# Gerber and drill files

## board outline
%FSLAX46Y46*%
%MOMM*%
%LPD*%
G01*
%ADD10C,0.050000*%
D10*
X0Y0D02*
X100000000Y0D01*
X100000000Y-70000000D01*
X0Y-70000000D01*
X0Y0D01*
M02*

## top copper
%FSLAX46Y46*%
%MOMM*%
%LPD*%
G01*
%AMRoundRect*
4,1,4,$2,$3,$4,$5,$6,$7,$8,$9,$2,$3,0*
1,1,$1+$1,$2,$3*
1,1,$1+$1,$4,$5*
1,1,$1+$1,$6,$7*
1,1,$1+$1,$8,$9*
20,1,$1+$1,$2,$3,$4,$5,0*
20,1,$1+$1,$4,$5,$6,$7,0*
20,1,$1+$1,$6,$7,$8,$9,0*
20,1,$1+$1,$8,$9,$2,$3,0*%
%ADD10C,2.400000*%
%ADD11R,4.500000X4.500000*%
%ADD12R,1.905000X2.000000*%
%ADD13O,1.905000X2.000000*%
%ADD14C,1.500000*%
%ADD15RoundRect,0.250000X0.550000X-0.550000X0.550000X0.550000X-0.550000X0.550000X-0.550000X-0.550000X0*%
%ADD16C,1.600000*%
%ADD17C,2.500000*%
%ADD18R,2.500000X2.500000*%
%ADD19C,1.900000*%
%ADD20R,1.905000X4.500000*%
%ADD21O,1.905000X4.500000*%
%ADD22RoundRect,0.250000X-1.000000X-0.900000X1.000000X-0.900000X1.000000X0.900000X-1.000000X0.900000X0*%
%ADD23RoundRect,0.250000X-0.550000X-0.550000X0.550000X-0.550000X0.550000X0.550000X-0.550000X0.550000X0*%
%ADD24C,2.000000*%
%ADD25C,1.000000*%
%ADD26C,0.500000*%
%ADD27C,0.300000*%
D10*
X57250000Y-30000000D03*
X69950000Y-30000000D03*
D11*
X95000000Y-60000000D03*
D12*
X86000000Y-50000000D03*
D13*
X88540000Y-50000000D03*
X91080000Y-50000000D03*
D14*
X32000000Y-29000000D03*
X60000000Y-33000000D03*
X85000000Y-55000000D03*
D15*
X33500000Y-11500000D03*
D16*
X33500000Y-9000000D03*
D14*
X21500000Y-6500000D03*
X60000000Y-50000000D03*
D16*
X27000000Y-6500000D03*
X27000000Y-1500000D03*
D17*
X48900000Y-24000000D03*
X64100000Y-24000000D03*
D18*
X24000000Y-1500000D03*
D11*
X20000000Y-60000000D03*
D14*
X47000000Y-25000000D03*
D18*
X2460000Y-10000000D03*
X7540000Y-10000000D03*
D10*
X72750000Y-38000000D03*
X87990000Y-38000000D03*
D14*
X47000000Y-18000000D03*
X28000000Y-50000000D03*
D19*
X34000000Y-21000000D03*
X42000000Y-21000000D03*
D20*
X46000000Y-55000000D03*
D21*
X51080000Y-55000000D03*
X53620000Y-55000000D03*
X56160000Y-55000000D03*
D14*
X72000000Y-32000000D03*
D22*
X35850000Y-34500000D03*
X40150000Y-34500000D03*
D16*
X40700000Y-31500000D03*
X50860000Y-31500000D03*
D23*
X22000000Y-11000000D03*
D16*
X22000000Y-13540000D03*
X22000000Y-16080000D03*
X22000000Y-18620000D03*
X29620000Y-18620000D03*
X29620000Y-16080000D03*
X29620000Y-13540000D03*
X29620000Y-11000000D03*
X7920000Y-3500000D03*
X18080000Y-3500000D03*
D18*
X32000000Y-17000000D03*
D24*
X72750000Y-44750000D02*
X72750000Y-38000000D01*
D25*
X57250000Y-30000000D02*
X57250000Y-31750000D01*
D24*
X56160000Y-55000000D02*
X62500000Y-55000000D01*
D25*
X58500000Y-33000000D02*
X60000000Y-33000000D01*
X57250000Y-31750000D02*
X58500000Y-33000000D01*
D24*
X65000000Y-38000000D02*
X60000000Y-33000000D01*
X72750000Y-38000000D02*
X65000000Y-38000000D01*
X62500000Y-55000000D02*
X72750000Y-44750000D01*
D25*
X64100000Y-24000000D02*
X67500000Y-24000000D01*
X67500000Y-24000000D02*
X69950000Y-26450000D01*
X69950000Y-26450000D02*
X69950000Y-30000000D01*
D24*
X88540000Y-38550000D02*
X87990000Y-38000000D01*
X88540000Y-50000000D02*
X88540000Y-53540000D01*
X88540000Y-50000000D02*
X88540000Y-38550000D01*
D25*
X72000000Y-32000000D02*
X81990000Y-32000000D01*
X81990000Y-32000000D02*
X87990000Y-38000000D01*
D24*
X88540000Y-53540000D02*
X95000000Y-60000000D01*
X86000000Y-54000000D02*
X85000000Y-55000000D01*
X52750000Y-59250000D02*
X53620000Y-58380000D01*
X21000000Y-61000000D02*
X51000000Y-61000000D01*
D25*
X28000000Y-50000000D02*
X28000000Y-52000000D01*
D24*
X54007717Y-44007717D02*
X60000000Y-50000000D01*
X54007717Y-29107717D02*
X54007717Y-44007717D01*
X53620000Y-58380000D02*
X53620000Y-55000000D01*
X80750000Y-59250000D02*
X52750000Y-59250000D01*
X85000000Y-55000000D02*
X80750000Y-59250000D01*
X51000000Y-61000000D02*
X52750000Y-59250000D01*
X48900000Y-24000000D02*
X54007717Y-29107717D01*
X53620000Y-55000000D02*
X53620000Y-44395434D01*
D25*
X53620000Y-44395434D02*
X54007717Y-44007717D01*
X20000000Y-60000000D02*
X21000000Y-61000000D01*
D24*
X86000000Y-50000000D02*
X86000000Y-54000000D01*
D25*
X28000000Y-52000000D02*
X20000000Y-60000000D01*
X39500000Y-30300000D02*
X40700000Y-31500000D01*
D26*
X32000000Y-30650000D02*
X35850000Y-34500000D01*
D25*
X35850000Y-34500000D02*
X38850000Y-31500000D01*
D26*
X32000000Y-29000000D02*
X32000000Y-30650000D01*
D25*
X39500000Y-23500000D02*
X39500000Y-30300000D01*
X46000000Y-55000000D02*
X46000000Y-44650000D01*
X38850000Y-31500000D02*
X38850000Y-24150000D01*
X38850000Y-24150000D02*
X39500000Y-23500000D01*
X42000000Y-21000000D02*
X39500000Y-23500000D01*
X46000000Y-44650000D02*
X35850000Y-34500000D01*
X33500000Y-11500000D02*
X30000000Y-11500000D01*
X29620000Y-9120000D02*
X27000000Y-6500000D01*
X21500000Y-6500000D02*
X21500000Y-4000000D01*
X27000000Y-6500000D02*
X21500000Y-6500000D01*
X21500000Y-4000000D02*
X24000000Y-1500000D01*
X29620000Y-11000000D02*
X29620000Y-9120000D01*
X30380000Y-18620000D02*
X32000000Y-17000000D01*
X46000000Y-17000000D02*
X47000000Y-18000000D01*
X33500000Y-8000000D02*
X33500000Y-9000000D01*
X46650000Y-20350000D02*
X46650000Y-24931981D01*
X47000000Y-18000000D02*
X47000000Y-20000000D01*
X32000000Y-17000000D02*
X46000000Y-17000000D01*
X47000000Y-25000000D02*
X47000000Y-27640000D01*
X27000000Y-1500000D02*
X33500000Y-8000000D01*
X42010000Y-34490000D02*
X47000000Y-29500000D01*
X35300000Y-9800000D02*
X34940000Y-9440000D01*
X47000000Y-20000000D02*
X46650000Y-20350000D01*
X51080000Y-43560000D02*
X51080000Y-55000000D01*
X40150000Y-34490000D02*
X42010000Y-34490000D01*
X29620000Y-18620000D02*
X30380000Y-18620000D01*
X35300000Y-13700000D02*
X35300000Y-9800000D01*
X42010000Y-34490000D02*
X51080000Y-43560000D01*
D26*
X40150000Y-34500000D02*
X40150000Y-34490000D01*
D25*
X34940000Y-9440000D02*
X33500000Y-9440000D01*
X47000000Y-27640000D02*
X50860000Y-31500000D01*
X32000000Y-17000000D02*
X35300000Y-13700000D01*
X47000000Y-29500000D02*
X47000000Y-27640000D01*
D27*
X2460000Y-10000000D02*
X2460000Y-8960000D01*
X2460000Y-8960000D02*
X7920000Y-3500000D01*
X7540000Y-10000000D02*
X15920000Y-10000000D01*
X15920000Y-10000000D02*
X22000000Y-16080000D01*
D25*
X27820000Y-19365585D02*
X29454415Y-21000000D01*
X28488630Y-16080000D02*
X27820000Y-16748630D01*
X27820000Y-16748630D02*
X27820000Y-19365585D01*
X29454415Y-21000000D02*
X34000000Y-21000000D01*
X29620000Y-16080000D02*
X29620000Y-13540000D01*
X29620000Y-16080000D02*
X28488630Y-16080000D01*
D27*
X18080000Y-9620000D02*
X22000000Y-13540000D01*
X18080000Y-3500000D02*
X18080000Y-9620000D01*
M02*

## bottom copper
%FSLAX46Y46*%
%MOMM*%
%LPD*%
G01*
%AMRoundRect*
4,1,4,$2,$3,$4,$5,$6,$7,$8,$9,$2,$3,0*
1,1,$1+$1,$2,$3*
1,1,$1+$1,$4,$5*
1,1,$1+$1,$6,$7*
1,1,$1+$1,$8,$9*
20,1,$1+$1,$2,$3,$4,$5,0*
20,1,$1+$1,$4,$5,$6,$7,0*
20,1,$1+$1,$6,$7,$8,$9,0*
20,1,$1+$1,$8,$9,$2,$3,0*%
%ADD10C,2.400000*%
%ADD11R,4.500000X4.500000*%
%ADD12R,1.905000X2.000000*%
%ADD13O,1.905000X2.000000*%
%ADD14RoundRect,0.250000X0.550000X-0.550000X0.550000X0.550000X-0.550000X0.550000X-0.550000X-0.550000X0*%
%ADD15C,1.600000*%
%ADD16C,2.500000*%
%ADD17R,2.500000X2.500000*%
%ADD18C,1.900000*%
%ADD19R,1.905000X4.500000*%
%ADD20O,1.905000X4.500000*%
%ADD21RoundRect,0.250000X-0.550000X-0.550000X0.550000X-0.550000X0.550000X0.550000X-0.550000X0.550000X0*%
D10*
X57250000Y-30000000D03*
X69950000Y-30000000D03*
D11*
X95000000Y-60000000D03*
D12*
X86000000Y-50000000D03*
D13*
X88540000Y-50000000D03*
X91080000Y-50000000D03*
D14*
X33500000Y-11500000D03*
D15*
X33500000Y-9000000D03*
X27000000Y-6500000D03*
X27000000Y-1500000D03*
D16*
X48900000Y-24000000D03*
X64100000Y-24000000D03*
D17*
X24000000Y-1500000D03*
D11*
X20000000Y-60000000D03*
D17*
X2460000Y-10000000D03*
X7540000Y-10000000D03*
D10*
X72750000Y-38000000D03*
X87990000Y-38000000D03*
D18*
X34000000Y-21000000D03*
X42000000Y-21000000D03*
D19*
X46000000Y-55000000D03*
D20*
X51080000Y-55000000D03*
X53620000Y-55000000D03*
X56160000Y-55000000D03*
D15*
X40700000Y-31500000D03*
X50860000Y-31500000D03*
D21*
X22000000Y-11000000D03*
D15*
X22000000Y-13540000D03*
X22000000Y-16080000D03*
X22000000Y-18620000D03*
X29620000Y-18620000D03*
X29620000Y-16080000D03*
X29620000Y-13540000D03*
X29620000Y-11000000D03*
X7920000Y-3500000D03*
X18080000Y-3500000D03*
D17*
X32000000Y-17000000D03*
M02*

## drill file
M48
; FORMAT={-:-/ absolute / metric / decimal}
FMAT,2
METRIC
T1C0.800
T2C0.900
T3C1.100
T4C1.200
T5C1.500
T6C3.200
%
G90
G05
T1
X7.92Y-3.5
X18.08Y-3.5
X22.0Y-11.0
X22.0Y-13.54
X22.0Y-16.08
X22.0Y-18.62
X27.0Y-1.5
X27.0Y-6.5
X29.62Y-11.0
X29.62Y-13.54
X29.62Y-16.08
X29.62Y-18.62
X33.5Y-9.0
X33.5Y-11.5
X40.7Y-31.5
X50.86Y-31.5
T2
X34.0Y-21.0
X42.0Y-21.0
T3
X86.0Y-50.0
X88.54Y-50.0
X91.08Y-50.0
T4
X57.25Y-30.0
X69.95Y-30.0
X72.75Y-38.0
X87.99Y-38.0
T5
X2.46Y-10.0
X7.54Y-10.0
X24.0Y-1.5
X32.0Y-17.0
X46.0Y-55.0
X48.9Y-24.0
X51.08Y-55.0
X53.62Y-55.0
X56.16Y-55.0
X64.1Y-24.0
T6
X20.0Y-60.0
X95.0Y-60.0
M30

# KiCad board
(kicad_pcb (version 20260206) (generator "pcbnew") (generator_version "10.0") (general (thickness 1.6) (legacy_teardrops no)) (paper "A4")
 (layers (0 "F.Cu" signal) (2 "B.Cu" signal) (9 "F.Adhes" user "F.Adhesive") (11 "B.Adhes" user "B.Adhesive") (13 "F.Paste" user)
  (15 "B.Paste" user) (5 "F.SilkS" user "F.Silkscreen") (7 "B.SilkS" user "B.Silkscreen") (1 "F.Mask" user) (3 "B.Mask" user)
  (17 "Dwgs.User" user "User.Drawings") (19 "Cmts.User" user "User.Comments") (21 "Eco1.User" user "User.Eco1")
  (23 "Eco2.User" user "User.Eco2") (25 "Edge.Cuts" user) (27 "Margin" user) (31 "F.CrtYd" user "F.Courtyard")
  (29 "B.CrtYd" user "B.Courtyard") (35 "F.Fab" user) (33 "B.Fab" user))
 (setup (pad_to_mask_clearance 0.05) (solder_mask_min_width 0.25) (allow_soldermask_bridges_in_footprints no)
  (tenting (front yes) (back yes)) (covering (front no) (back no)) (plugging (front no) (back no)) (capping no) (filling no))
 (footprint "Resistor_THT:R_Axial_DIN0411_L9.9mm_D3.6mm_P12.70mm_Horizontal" (layer "F.Cu") (at 57.25 30)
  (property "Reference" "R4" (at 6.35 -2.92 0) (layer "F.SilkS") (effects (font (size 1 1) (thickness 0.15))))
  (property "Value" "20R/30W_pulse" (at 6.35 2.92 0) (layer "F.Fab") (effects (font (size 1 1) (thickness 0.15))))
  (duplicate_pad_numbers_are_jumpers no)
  (pad "1" thru_hole circle (at 0 0) (size 2.4 2.4) (drill 1.2) (layers "*.Cu" "*.Mask") (remove_unused_layers no) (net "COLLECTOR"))
  (pad "2" thru_hole circle (at 12.7 0) (size 2.4 2.4) (drill 1.2) (layers "*.Cu" "*.Mask") (remove_unused_layers no)
   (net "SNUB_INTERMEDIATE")))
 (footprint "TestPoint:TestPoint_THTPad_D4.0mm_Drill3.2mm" (layer "F.Cu") (at 95 60)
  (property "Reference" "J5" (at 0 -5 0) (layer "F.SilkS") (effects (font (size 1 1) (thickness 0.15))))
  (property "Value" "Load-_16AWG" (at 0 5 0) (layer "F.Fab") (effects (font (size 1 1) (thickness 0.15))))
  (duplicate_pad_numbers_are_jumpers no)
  (pad "1" thru_hole rect (at 0 0) (size 4.5 4.5) (drill 3.2) (layers "*.Cu" "*.Mask") (remove_unused_layers no) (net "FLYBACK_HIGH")))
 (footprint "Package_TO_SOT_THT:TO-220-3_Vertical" (layer "F.Cu") (at 86 50)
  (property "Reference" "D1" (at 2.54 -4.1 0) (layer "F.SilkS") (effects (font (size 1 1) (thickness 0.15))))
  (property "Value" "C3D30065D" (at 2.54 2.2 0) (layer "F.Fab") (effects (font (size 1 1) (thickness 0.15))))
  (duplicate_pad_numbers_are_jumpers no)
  (pad "1" thru_hole rect (at 0 0) (size 1.905 2) (drill 1.1) (layers "*.Cu" "*.Mask") (remove_unused_layers no) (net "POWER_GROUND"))
  (pad "2" thru_hole oval (at 2.54 0) (size 1.905 2) (drill 1.1) (layers "*.Cu" "*.Mask") (remove_unused_layers no) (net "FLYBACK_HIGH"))
  (pad "3" thru_hole oval (at 5.08 0) (size 1.905 2) (drill 1.1) (layers "*.Cu" "*.Mask") (remove_unused_layers no) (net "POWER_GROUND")))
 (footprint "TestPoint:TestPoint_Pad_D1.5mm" (layer "F.Cu") (at 32 29)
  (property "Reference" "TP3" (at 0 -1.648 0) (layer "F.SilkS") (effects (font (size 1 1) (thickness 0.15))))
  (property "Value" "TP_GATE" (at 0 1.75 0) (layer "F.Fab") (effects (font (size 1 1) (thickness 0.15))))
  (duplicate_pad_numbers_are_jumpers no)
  (pad "1" smd circle (at 0 0) (size 1.5 1.5) (layers "F.Cu" "F.Mask") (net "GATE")))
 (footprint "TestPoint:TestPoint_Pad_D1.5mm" (layer "F.Cu") (at 60 33)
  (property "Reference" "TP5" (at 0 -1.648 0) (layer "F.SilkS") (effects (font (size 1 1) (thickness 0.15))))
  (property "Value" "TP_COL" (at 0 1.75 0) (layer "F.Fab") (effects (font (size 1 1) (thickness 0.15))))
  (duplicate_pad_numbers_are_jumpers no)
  (pad "1" smd circle (at 0 0) (size 1.5 1.5) (layers "F.Cu" "F.Mask") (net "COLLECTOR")))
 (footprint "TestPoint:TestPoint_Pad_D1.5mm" (layer "F.Cu") (at 85 55)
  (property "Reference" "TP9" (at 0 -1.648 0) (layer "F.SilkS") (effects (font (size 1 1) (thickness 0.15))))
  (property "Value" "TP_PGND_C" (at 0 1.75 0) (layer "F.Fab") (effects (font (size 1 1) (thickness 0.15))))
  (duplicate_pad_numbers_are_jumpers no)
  (pad "1" smd circle (at 0 0) (size 1.5 1.5) (layers "F.Cu" "F.Mask") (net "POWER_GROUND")))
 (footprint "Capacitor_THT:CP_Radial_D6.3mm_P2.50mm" (layer "F.Cu") (at 33.5 11.5 90)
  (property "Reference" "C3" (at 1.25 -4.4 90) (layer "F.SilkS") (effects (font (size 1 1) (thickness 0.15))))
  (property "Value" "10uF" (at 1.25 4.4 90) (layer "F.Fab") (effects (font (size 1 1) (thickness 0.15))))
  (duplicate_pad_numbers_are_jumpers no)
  (pad "1" thru_hole roundrect (at 0 0 90) (size 1.6 1.6) (drill 0.8) (layers "*.Cu" "*.Mask") (remove_unused_layers no)
   (roundrect_rratio 0.15625) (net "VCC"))
  (pad "2" thru_hole circle (at 2.5 0 90) (size 1.6 1.6) (drill 0.8) (layers "*.Cu" "*.Mask") (remove_unused_layers no)
   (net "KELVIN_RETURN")))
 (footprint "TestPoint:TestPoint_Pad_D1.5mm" (layer "F.Cu") (at 21.5 6.5)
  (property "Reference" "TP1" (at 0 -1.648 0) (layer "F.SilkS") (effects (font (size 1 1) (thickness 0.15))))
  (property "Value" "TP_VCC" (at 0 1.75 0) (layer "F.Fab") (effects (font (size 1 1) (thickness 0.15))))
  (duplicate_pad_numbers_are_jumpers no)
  (pad "1" smd circle (at 0 0) (size 1.5 1.5) (layers "F.Cu" "F.Mask") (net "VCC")))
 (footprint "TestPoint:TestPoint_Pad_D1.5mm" (layer "F.Cu") (at 60 50)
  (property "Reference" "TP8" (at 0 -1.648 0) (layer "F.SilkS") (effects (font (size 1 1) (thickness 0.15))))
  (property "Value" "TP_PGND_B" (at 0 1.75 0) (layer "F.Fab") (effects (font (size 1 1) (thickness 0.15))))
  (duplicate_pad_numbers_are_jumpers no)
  (pad "1" smd circle (at 0 0) (size 1.5 1.5) (layers "F.Cu" "F.Mask") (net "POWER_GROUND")))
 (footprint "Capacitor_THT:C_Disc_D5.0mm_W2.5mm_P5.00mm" (layer "F.Cu") (at 27 6.5 90)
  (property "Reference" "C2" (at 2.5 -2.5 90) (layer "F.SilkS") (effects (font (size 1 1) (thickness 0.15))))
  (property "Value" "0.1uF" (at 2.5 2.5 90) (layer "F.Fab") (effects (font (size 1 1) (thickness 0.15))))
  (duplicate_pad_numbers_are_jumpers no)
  (pad "1" thru_hole circle (at 0 0 90) (size 1.6 1.6) (drill 0.8) (layers "*.Cu" "*.Mask") (remove_unused_layers no) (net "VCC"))
  (pad "2" thru_hole circle (at 5 0 90) (size 1.6 1.6) (drill 0.8) (layers "*.Cu" "*.Mask") (remove_unused_layers no) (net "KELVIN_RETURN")))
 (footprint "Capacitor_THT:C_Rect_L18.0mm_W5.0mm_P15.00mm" (layer "F.Cu") (at 56.5 24)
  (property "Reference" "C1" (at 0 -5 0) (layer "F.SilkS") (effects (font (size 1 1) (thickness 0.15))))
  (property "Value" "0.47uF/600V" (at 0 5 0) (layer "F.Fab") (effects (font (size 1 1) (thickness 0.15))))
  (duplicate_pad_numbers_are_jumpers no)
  (pad "1" thru_hole circle (at -7.6 0) (size 2.5 2.5) (drill 1.5) (layers "*.Cu" "*.Mask") (remove_unused_layers no) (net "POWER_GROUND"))
  (pad "2" thru_hole circle (at 7.6 0) (size 2.5 2.5) (drill 1.5) (layers "*.Cu" "*.Mask") (remove_unused_layers no)
   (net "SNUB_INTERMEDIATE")))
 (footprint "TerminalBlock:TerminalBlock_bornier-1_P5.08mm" (layer "F.Cu") (at 24 1.5)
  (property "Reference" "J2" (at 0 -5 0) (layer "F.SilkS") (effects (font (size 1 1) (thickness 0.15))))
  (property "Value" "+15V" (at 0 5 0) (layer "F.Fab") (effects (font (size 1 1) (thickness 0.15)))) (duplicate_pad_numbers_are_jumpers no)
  (pad "1" thru_hole rect (at 0 0) (size 2.5 2.5) (drill 1.5) (layers "*.Cu" "*.Mask") (remove_unused_layers no) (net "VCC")))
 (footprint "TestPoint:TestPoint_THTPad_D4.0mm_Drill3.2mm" (layer "F.Cu") (at 20 60)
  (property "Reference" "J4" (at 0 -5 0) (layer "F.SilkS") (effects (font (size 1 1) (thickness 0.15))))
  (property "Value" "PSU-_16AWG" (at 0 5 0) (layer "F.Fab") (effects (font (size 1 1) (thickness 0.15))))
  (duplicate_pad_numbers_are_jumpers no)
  (pad "1" thru_hole rect (at 0 0) (size 4.5 4.5) (drill 3.2) (layers "*.Cu" "*.Mask") (remove_unused_layers no) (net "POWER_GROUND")))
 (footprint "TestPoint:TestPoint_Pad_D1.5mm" (layer "F.Cu") (at 47 25)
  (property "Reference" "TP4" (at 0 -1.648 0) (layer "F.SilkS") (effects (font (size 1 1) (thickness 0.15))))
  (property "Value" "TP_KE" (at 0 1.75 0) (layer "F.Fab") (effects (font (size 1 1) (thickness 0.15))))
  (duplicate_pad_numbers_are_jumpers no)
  (pad "1" smd circle (at 0 0) (size 1.5 1.5) (layers "F.Cu" "F.Mask") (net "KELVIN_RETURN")))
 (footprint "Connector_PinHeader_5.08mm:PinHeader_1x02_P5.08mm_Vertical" (layer "F.Cu") (at 5 10 90)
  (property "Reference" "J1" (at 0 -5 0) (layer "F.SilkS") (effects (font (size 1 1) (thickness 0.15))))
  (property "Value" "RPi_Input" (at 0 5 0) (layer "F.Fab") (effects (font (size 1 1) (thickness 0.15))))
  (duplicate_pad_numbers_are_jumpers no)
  (pad "1" thru_hole rect (at 0 -2.54) (size 2.5 2.5) (drill 1.5) (layers "*.Cu" "*.Mask") (remove_unused_layers no) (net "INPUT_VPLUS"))
  (pad "2" thru_hole rect (at 0 2.54) (size 2.5 2.5) (drill 1.5) (layers "*.Cu" "*.Mask") (remove_unused_layers no) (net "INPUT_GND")))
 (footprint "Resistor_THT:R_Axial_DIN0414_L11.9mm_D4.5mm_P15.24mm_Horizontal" (layer "F.Cu") (at 72.75 38)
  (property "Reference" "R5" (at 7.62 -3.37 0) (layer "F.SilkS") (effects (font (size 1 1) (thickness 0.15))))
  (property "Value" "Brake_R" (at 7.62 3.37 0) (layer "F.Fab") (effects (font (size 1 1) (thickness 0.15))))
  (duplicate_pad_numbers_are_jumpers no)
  (pad "1" thru_hole circle (at 0 0) (size 2.4 2.4) (drill 1.2) (layers "*.Cu" "*.Mask") (remove_unused_layers no) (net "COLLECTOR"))
  (pad "2" thru_hole circle (at 15.24 0) (size 2.4 2.4) (drill 1.2) (layers "*.Cu" "*.Mask") (remove_unused_layers no) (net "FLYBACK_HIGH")))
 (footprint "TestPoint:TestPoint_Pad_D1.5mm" (layer "F.Cu") (at 47 18)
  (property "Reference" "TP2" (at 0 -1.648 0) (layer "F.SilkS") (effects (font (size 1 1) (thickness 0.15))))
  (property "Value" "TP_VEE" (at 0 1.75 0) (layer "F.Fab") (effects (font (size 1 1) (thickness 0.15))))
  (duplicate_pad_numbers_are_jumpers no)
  (pad "1" smd circle (at 0 0) (size 1.5 1.5) (layers "F.Cu" "F.Mask") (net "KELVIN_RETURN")))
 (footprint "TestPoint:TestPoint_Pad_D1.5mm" (layer "F.Cu") (at 28 50)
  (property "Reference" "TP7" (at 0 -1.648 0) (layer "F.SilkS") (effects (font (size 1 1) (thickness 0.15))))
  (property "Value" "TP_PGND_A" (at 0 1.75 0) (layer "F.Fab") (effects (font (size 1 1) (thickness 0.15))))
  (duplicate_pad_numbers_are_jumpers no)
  (pad "1" smd circle (at 0 0) (size 1.5 1.5) (layers "F.Cu" "F.Mask") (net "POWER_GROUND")))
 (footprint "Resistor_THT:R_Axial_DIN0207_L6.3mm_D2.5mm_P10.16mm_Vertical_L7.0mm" (layer "F.Cu") (at 38 21 90)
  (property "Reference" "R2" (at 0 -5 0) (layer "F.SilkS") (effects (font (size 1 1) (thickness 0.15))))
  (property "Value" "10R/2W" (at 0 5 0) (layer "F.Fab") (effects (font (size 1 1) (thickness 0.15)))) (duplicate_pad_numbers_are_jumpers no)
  (pad "1" thru_hole circle (at 0 -4) (size 1.9 1.9) (drill 0.9) (layers "*.Cu" "*.Mask") (remove_unused_layers no) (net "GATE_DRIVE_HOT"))
  (pad "2" thru_hole circle (at 0 4) (size 1.9 1.9) (drill 0.9) (layers "*.Cu" "*.Mask") (remove_unused_layers no) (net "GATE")))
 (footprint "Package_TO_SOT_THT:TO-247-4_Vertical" (layer "F.Cu") (at 46 55)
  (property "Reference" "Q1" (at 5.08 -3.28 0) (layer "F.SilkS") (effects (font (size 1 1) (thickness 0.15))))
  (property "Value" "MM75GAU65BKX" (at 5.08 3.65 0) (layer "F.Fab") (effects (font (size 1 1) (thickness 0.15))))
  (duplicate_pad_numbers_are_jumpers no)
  (pad "1" thru_hole rect (at 0 0) (size 1.905 4.5) (drill 1.5) (layers "*.Cu" "*.Mask") (remove_unused_layers no) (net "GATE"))
  (pad "2" thru_hole oval (at 5.08 0) (size 1.905 4.5) (drill 1.5) (layers "*.Cu" "*.Mask") (remove_unused_layers no) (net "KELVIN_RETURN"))
  (pad "3" thru_hole oval (at 7.62 0) (size 1.905 4.5) (drill 1.5) (layers "*.Cu" "*.Mask") (remove_unused_layers no) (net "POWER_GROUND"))
  (pad "4" thru_hole oval (at 10.16 0) (size 1.905 4.5) (drill 1.5) (layers "*.Cu" "*.Mask") (remove_unused_layers no) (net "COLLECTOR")))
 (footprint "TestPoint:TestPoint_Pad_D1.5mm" (layer "F.Cu") (at 72 32)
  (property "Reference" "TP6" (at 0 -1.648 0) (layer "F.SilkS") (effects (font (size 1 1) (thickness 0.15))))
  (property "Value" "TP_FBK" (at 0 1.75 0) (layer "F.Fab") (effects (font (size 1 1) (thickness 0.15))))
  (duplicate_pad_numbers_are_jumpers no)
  (pad "1" smd circle (at 0 0) (size 1.5 1.5) (layers "F.Cu" "F.Mask") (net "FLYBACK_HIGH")))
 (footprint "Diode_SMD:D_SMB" (layer "F.Cu") (at 38 34.5)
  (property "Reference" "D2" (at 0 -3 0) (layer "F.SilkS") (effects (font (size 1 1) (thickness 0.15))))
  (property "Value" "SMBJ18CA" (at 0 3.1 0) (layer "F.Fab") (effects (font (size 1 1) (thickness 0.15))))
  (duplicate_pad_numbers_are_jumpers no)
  (pad "1" smd roundrect (at -2.15 0) (size 2.5 2.3) (layers "F.Cu" "F.Mask" "F.Paste") (roundrect_rratio 0.1086956522) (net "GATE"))
  (pad "2" smd roundrect (at 2.15 0) (size 2.5 2.3) (layers "F.Cu" "F.Mask" "F.Paste") (roundrect_rratio 0.1086956522) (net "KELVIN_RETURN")))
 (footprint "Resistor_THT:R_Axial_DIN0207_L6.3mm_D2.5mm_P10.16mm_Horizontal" (layer "F.Cu") (at 40.7 31.5)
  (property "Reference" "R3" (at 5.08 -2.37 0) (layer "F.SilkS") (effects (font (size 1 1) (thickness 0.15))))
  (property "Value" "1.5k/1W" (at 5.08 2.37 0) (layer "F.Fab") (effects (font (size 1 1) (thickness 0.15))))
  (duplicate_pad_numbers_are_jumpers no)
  (pad "1" thru_hole circle (at 0 0) (size 1.6 1.6) (drill 0.8) (layers "*.Cu" "*.Mask") (remove_unused_layers no) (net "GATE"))
  (pad "2" thru_hole circle (at 10.16 0) (size 1.6 1.6) (drill 0.8) (layers "*.Cu" "*.Mask") (remove_unused_layers no) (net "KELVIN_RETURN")))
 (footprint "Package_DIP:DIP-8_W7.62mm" (layer "F.Cu") (at 22 11)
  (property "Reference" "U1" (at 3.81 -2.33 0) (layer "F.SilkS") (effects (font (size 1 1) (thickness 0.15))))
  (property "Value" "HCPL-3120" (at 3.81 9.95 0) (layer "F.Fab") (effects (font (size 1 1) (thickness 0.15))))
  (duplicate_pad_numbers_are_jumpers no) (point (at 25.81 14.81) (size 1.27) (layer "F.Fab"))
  (pad "1" thru_hole roundrect (at 0 0) (size 1.6 1.6) (drill 0.8) (layers "*.Cu" "*.Mask") (remove_unused_layers no)
   (roundrect_rratio 0.15625))
  (pad "2" thru_hole circle (at 0 2.54) (size 1.6 1.6) (drill 0.8) (layers "*.Cu" "*.Mask") (remove_unused_layers no) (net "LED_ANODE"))
  (pad "3" thru_hole circle (at 0 5.08) (size 1.6 1.6) (drill 0.8) (layers "*.Cu" "*.Mask") (remove_unused_layers no) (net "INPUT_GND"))
  (pad "4" thru_hole circle (at 0 7.62) (size 1.6 1.6) (drill 0.8) (layers "*.Cu" "*.Mask") (remove_unused_layers no))
  (pad "5" thru_hole circle (at 7.62 7.62) (size 1.6 1.6) (drill 0.8) (layers "*.Cu" "*.Mask") (remove_unused_layers no)
   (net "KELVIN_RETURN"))
  (pad "6" thru_hole circle (at 7.62 5.08) (size 1.6 1.6) (drill 0.8) (layers "*.Cu" "*.Mask") (remove_unused_layers no)
   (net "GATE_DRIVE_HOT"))
  (pad "7" thru_hole circle (at 7.62 2.54) (size 1.6 1.6) (drill 0.8) (layers "*.Cu" "*.Mask") (remove_unused_layers no)
   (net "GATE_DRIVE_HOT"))
  (pad "8" thru_hole circle (at 7.62 0) (size 1.6 1.6) (drill 0.8) (layers "*.Cu" "*.Mask") (remove_unused_layers no) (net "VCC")))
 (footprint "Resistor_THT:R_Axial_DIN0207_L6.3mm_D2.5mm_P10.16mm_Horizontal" (layer "F.Cu") (at 7.92 3.5)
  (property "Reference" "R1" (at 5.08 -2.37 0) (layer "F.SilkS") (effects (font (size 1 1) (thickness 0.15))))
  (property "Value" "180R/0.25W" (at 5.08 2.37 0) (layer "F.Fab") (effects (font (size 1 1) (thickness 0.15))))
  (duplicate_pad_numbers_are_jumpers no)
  (pad "1" thru_hole circle (at 0 0) (size 1.6 1.6) (drill 0.8) (layers "*.Cu" "*.Mask") (remove_unused_layers no) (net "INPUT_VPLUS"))
  (pad "2" thru_hole circle (at 10.16 0) (size 1.6 1.6) (drill 0.8) (layers "*.Cu" "*.Mask") (remove_unused_layers no) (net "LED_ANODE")))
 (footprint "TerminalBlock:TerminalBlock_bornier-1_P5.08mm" (layer "F.Cu") (at 32 17)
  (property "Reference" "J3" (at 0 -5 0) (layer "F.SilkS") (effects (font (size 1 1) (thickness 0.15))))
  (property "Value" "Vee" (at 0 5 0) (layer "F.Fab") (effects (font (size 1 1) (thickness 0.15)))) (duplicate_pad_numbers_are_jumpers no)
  (pad "1" thru_hole rect (at 0 0) (size 2.5 2.5) (drill 1.5) (layers "*.Cu" "*.Mask") (remove_unused_layers no) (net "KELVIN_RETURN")))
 (gr_rect (start 0 0) (end 100 70) (stroke (width 0.05) (type solid)) (fill no) (layer "Edge.Cuts"))
 (segment (start 72.75 44.75) (end 72.75 38) (width 2) (layer "F.Cu") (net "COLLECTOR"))
 (segment (start 57.25 30) (end 57.25 31.75) (width 1) (layer "F.Cu") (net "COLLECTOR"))
 (segment (start 56.16 55) (end 62.5 55) (width 2) (layer "F.Cu") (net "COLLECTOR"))
 (segment (start 58.5 33) (end 60 33) (width 1) (layer "F.Cu") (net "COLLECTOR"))
 (segment (start 57.25 31.75) (end 58.5 33) (width 1) (layer "F.Cu") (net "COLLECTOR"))
 (segment (start 65 38) (end 60 33) (width 2) (layer "F.Cu") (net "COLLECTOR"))
 (segment (start 72.75 38) (end 65 38) (width 2) (layer "F.Cu") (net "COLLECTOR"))
 (segment (start 62.5 55) (end 72.75 44.75) (width 2) (layer "F.Cu") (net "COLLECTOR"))
 (segment (start 64.1 24) (end 67.5 24) (width 1) (layer "F.Cu") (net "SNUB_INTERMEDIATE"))
 (segment (start 67.5 24) (end 69.95 26.45) (width 1) (layer "F.Cu") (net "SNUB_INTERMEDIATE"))
 (segment (start 69.95 26.45) (end 69.95 30) (width 1) (layer "F.Cu") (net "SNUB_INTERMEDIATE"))
 (segment (start 88.54 38.55) (end 87.99 38) (width 2) (layer "F.Cu") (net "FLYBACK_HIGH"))
 (segment (start 88.54 50) (end 88.54 53.54) (width 2) (layer "F.Cu") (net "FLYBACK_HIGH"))
 (segment (start 88.54 50) (end 88.54 38.55) (width 2) (layer "F.Cu") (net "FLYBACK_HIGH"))
 (segment (start 72 32) (end 81.99 32) (width 1) (layer "F.Cu") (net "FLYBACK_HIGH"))
 (segment (start 81.99 32) (end 87.99 38) (width 1) (layer "F.Cu") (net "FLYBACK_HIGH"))
 (segment (start 88.54 53.54) (end 95 60) (width 2) (layer "F.Cu") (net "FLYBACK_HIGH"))
 (segment (start 86 54) (end 85 55) (width 2) (layer "F.Cu") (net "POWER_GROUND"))
 (segment (start 52.75 59.25) (end 53.62 58.38) (width 2) (layer "F.Cu") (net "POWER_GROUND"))
 (segment (start 21 61) (end 51 61) (width 2) (layer "F.Cu") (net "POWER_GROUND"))
 (segment (start 28 50) (end 28 52) (width 1) (layer "F.Cu") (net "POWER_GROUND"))
 (segment (start 54.007717 44.007717) (end 60 50) (width 2) (layer "F.Cu") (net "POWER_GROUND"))
 (segment (start 54.007717 29.107717) (end 54.007717 44.007717) (width 2) (layer "F.Cu") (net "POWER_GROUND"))
 (segment (start 53.62 58.38) (end 53.62 55) (width 2) (layer "F.Cu") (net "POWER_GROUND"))
 (segment (start 80.75 59.25) (end 52.75 59.25) (width 2) (layer "F.Cu") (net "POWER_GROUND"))
 (segment (start 85 55) (end 80.75 59.25) (width 2) (layer "F.Cu") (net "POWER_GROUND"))
 (segment (start 51 61) (end 52.75 59.25) (width 2) (layer "F.Cu") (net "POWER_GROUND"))
 (segment (start 48.9 24) (end 54.007717 29.107717) (width 2) (layer "F.Cu") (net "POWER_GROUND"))
 (segment (start 53.62 55) (end 53.62 44.395434) (width 2) (layer "F.Cu") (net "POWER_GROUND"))
 (segment (start 53.62 44.395434) (end 54.007717 44.007717) (width 1) (layer "F.Cu") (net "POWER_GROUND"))
 (segment (start 20 60) (end 21 61) (width 1) (layer "F.Cu") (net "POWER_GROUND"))
 (segment (start 86 50) (end 86 54) (width 2) (layer "F.Cu") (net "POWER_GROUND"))
 (segment (start 28 52) (end 20 60) (width 1) (layer "F.Cu") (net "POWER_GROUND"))
 (segment (start 39.5 30.3) (end 40.7 31.5) (width 1) (layer "F.Cu") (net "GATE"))
 (segment (start 32 30.65) (end 35.85 34.5) (width 0.5) (layer "F.Cu") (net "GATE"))
 (segment (start 35.85 34.5) (end 38.85 31.5) (width 1) (layer "F.Cu") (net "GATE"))
 (segment (start 32 29) (end 32 30.65) (width 0.5) (layer "F.Cu") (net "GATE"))
 (segment (start 39.5 23.5) (end 39.5 30.3) (width 1) (layer "F.Cu") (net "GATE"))
 (segment (start 46 55) (end 46 44.65) (width 1) (layer "F.Cu") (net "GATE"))
 (segment (start 38.85 31.5) (end 38.85 24.15) (width 1) (layer "F.Cu") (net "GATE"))
 (segment (start 38.85 24.15) (end 39.5 23.5) (width 1) (layer "F.Cu") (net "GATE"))
 (segment (start 42 21) (end 39.5 23.5) (width 1) (layer "F.Cu") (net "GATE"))
 (segment (start 46 44.65) (end 35.85 34.5) (width 1) (layer "F.Cu") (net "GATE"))
 (segment (start 33.5 11.5) (end 30 11.5) (width 1) (layer "F.Cu") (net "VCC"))
 (segment (start 29.62 9.12) (end 27 6.5) (width 1) (layer "F.Cu") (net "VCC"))
 (segment (start 21.5 6.5) (end 21.5 4) (width 1) (layer "F.Cu") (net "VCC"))
 (segment (start 27 6.5) (end 21.5 6.5) (width 1) (layer "F.Cu") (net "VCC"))
 (segment (start 21.5 4) (end 24 1.5) (width 1) (layer "F.Cu") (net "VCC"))
 (segment (start 29.62 11) (end 29.62 9.12) (width 1) (layer "F.Cu") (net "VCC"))
 (segment (start 30.38 18.62) (end 32 17) (width 1) (layer "F.Cu") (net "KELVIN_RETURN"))
 (segment (start 46 17) (end 47 18) (width 1) (layer "F.Cu") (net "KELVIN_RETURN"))
 (segment (start 33.5 8) (end 33.5 9) (width 1) (layer "F.Cu") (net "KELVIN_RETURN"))
 (segment (start 46.65 20.35) (end 46.65 24.931981) (width 1) (layer "F.Cu") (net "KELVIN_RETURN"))
 (segment (start 47 18) (end 47 20) (width 1) (layer "F.Cu") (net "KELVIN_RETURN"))
 (segment (start 32 17) (end 46 17) (width 1) (layer "F.Cu") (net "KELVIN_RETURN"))
 (segment (start 47 25) (end 47 27.64) (width 1) (layer "F.Cu") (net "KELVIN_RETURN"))
 (segment (start 27 1.5) (end 33.5 8) (width 1) (layer "F.Cu") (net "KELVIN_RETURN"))
 (segment (start 42.01 34.49) (end 47 29.5) (width 1) (layer "F.Cu") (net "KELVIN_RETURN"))
 (segment (start 35.3 9.8) (end 34.94 9.44) (width 1) (layer "F.Cu") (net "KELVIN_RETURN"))
 (segment (start 47 20) (end 46.65 20.35) (width 1) (layer "F.Cu") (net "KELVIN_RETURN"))
 (segment (start 51.08 43.56) (end 51.08 55) (width 1) (layer "F.Cu") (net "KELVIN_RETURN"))
 (segment (start 40.15 34.49) (end 42.01 34.49) (width 1) (layer "F.Cu") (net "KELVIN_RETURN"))
 (segment (start 29.62 18.62) (end 30.38 18.62) (width 1) (layer "F.Cu") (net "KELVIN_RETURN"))
 (segment (start 35.3 13.7) (end 35.3 9.8) (width 1) (layer "F.Cu") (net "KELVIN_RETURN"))
 (segment (start 42.01 34.49) (end 51.08 43.56) (width 1) (layer "F.Cu") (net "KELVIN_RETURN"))
 (segment (start 40.15 34.5) (end 40.15 34.49) (width 0.5) (layer "F.Cu") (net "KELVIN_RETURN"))
 (segment (start 34.94 9.44) (end 33.5 9.44) (width 1) (layer "F.Cu") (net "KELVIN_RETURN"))
 (segment (start 47 27.64) (end 50.86 31.5) (width 1) (layer "F.Cu") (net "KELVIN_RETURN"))
 (segment (start 32 17) (end 35.3 13.7) (width 1) (layer "F.Cu") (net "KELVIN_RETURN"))
 (segment (start 47 29.5) (end 47 27.64) (width 1) (layer "F.Cu") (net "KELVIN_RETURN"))
 (segment (start 2.46 10) (end 2.46 8.96) (width 0.3) (layer "F.Cu") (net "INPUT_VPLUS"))
 (segment (start 2.46 8.96) (end 7.92 3.5) (width 0.3) (layer "F.Cu") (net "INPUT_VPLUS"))
 (segment (start 7.54 10) (end 15.92 10) (width 0.3) (layer "F.Cu") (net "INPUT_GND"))
 (segment (start 15.92 10) (end 22 16.08) (width 0.3) (layer "F.Cu") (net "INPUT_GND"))
 (segment (start 27.82 19.365585) (end 29.454415 21) (width 1) (layer "F.Cu") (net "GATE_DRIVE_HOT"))
 (segment (start 28.48863 16.08) (end 27.82 16.74863) (width 1) (layer "F.Cu") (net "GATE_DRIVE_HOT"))
 (segment (start 27.82 16.74863) (end 27.82 19.365585) (width 1) (layer "F.Cu") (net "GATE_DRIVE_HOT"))
 (segment (start 29.454415 21) (end 34 21) (width 1) (layer "F.Cu") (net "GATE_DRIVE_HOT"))
 (segment (start 29.62 16.08) (end 29.62 13.54) (width 1) (layer "F.Cu") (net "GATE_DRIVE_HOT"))
 (segment (start 29.62 16.08) (end 28.48863 16.08) (width 1) (layer "F.Cu") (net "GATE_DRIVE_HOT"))
 (segment (start 18.08 9.62) (end 22 13.54) (width 0.3) (layer "F.Cu") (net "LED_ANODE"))
 (segment (start 18.08 3.5) (end 18.08 9.62) (width 0.3) (layer "F.Cu") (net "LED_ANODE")))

